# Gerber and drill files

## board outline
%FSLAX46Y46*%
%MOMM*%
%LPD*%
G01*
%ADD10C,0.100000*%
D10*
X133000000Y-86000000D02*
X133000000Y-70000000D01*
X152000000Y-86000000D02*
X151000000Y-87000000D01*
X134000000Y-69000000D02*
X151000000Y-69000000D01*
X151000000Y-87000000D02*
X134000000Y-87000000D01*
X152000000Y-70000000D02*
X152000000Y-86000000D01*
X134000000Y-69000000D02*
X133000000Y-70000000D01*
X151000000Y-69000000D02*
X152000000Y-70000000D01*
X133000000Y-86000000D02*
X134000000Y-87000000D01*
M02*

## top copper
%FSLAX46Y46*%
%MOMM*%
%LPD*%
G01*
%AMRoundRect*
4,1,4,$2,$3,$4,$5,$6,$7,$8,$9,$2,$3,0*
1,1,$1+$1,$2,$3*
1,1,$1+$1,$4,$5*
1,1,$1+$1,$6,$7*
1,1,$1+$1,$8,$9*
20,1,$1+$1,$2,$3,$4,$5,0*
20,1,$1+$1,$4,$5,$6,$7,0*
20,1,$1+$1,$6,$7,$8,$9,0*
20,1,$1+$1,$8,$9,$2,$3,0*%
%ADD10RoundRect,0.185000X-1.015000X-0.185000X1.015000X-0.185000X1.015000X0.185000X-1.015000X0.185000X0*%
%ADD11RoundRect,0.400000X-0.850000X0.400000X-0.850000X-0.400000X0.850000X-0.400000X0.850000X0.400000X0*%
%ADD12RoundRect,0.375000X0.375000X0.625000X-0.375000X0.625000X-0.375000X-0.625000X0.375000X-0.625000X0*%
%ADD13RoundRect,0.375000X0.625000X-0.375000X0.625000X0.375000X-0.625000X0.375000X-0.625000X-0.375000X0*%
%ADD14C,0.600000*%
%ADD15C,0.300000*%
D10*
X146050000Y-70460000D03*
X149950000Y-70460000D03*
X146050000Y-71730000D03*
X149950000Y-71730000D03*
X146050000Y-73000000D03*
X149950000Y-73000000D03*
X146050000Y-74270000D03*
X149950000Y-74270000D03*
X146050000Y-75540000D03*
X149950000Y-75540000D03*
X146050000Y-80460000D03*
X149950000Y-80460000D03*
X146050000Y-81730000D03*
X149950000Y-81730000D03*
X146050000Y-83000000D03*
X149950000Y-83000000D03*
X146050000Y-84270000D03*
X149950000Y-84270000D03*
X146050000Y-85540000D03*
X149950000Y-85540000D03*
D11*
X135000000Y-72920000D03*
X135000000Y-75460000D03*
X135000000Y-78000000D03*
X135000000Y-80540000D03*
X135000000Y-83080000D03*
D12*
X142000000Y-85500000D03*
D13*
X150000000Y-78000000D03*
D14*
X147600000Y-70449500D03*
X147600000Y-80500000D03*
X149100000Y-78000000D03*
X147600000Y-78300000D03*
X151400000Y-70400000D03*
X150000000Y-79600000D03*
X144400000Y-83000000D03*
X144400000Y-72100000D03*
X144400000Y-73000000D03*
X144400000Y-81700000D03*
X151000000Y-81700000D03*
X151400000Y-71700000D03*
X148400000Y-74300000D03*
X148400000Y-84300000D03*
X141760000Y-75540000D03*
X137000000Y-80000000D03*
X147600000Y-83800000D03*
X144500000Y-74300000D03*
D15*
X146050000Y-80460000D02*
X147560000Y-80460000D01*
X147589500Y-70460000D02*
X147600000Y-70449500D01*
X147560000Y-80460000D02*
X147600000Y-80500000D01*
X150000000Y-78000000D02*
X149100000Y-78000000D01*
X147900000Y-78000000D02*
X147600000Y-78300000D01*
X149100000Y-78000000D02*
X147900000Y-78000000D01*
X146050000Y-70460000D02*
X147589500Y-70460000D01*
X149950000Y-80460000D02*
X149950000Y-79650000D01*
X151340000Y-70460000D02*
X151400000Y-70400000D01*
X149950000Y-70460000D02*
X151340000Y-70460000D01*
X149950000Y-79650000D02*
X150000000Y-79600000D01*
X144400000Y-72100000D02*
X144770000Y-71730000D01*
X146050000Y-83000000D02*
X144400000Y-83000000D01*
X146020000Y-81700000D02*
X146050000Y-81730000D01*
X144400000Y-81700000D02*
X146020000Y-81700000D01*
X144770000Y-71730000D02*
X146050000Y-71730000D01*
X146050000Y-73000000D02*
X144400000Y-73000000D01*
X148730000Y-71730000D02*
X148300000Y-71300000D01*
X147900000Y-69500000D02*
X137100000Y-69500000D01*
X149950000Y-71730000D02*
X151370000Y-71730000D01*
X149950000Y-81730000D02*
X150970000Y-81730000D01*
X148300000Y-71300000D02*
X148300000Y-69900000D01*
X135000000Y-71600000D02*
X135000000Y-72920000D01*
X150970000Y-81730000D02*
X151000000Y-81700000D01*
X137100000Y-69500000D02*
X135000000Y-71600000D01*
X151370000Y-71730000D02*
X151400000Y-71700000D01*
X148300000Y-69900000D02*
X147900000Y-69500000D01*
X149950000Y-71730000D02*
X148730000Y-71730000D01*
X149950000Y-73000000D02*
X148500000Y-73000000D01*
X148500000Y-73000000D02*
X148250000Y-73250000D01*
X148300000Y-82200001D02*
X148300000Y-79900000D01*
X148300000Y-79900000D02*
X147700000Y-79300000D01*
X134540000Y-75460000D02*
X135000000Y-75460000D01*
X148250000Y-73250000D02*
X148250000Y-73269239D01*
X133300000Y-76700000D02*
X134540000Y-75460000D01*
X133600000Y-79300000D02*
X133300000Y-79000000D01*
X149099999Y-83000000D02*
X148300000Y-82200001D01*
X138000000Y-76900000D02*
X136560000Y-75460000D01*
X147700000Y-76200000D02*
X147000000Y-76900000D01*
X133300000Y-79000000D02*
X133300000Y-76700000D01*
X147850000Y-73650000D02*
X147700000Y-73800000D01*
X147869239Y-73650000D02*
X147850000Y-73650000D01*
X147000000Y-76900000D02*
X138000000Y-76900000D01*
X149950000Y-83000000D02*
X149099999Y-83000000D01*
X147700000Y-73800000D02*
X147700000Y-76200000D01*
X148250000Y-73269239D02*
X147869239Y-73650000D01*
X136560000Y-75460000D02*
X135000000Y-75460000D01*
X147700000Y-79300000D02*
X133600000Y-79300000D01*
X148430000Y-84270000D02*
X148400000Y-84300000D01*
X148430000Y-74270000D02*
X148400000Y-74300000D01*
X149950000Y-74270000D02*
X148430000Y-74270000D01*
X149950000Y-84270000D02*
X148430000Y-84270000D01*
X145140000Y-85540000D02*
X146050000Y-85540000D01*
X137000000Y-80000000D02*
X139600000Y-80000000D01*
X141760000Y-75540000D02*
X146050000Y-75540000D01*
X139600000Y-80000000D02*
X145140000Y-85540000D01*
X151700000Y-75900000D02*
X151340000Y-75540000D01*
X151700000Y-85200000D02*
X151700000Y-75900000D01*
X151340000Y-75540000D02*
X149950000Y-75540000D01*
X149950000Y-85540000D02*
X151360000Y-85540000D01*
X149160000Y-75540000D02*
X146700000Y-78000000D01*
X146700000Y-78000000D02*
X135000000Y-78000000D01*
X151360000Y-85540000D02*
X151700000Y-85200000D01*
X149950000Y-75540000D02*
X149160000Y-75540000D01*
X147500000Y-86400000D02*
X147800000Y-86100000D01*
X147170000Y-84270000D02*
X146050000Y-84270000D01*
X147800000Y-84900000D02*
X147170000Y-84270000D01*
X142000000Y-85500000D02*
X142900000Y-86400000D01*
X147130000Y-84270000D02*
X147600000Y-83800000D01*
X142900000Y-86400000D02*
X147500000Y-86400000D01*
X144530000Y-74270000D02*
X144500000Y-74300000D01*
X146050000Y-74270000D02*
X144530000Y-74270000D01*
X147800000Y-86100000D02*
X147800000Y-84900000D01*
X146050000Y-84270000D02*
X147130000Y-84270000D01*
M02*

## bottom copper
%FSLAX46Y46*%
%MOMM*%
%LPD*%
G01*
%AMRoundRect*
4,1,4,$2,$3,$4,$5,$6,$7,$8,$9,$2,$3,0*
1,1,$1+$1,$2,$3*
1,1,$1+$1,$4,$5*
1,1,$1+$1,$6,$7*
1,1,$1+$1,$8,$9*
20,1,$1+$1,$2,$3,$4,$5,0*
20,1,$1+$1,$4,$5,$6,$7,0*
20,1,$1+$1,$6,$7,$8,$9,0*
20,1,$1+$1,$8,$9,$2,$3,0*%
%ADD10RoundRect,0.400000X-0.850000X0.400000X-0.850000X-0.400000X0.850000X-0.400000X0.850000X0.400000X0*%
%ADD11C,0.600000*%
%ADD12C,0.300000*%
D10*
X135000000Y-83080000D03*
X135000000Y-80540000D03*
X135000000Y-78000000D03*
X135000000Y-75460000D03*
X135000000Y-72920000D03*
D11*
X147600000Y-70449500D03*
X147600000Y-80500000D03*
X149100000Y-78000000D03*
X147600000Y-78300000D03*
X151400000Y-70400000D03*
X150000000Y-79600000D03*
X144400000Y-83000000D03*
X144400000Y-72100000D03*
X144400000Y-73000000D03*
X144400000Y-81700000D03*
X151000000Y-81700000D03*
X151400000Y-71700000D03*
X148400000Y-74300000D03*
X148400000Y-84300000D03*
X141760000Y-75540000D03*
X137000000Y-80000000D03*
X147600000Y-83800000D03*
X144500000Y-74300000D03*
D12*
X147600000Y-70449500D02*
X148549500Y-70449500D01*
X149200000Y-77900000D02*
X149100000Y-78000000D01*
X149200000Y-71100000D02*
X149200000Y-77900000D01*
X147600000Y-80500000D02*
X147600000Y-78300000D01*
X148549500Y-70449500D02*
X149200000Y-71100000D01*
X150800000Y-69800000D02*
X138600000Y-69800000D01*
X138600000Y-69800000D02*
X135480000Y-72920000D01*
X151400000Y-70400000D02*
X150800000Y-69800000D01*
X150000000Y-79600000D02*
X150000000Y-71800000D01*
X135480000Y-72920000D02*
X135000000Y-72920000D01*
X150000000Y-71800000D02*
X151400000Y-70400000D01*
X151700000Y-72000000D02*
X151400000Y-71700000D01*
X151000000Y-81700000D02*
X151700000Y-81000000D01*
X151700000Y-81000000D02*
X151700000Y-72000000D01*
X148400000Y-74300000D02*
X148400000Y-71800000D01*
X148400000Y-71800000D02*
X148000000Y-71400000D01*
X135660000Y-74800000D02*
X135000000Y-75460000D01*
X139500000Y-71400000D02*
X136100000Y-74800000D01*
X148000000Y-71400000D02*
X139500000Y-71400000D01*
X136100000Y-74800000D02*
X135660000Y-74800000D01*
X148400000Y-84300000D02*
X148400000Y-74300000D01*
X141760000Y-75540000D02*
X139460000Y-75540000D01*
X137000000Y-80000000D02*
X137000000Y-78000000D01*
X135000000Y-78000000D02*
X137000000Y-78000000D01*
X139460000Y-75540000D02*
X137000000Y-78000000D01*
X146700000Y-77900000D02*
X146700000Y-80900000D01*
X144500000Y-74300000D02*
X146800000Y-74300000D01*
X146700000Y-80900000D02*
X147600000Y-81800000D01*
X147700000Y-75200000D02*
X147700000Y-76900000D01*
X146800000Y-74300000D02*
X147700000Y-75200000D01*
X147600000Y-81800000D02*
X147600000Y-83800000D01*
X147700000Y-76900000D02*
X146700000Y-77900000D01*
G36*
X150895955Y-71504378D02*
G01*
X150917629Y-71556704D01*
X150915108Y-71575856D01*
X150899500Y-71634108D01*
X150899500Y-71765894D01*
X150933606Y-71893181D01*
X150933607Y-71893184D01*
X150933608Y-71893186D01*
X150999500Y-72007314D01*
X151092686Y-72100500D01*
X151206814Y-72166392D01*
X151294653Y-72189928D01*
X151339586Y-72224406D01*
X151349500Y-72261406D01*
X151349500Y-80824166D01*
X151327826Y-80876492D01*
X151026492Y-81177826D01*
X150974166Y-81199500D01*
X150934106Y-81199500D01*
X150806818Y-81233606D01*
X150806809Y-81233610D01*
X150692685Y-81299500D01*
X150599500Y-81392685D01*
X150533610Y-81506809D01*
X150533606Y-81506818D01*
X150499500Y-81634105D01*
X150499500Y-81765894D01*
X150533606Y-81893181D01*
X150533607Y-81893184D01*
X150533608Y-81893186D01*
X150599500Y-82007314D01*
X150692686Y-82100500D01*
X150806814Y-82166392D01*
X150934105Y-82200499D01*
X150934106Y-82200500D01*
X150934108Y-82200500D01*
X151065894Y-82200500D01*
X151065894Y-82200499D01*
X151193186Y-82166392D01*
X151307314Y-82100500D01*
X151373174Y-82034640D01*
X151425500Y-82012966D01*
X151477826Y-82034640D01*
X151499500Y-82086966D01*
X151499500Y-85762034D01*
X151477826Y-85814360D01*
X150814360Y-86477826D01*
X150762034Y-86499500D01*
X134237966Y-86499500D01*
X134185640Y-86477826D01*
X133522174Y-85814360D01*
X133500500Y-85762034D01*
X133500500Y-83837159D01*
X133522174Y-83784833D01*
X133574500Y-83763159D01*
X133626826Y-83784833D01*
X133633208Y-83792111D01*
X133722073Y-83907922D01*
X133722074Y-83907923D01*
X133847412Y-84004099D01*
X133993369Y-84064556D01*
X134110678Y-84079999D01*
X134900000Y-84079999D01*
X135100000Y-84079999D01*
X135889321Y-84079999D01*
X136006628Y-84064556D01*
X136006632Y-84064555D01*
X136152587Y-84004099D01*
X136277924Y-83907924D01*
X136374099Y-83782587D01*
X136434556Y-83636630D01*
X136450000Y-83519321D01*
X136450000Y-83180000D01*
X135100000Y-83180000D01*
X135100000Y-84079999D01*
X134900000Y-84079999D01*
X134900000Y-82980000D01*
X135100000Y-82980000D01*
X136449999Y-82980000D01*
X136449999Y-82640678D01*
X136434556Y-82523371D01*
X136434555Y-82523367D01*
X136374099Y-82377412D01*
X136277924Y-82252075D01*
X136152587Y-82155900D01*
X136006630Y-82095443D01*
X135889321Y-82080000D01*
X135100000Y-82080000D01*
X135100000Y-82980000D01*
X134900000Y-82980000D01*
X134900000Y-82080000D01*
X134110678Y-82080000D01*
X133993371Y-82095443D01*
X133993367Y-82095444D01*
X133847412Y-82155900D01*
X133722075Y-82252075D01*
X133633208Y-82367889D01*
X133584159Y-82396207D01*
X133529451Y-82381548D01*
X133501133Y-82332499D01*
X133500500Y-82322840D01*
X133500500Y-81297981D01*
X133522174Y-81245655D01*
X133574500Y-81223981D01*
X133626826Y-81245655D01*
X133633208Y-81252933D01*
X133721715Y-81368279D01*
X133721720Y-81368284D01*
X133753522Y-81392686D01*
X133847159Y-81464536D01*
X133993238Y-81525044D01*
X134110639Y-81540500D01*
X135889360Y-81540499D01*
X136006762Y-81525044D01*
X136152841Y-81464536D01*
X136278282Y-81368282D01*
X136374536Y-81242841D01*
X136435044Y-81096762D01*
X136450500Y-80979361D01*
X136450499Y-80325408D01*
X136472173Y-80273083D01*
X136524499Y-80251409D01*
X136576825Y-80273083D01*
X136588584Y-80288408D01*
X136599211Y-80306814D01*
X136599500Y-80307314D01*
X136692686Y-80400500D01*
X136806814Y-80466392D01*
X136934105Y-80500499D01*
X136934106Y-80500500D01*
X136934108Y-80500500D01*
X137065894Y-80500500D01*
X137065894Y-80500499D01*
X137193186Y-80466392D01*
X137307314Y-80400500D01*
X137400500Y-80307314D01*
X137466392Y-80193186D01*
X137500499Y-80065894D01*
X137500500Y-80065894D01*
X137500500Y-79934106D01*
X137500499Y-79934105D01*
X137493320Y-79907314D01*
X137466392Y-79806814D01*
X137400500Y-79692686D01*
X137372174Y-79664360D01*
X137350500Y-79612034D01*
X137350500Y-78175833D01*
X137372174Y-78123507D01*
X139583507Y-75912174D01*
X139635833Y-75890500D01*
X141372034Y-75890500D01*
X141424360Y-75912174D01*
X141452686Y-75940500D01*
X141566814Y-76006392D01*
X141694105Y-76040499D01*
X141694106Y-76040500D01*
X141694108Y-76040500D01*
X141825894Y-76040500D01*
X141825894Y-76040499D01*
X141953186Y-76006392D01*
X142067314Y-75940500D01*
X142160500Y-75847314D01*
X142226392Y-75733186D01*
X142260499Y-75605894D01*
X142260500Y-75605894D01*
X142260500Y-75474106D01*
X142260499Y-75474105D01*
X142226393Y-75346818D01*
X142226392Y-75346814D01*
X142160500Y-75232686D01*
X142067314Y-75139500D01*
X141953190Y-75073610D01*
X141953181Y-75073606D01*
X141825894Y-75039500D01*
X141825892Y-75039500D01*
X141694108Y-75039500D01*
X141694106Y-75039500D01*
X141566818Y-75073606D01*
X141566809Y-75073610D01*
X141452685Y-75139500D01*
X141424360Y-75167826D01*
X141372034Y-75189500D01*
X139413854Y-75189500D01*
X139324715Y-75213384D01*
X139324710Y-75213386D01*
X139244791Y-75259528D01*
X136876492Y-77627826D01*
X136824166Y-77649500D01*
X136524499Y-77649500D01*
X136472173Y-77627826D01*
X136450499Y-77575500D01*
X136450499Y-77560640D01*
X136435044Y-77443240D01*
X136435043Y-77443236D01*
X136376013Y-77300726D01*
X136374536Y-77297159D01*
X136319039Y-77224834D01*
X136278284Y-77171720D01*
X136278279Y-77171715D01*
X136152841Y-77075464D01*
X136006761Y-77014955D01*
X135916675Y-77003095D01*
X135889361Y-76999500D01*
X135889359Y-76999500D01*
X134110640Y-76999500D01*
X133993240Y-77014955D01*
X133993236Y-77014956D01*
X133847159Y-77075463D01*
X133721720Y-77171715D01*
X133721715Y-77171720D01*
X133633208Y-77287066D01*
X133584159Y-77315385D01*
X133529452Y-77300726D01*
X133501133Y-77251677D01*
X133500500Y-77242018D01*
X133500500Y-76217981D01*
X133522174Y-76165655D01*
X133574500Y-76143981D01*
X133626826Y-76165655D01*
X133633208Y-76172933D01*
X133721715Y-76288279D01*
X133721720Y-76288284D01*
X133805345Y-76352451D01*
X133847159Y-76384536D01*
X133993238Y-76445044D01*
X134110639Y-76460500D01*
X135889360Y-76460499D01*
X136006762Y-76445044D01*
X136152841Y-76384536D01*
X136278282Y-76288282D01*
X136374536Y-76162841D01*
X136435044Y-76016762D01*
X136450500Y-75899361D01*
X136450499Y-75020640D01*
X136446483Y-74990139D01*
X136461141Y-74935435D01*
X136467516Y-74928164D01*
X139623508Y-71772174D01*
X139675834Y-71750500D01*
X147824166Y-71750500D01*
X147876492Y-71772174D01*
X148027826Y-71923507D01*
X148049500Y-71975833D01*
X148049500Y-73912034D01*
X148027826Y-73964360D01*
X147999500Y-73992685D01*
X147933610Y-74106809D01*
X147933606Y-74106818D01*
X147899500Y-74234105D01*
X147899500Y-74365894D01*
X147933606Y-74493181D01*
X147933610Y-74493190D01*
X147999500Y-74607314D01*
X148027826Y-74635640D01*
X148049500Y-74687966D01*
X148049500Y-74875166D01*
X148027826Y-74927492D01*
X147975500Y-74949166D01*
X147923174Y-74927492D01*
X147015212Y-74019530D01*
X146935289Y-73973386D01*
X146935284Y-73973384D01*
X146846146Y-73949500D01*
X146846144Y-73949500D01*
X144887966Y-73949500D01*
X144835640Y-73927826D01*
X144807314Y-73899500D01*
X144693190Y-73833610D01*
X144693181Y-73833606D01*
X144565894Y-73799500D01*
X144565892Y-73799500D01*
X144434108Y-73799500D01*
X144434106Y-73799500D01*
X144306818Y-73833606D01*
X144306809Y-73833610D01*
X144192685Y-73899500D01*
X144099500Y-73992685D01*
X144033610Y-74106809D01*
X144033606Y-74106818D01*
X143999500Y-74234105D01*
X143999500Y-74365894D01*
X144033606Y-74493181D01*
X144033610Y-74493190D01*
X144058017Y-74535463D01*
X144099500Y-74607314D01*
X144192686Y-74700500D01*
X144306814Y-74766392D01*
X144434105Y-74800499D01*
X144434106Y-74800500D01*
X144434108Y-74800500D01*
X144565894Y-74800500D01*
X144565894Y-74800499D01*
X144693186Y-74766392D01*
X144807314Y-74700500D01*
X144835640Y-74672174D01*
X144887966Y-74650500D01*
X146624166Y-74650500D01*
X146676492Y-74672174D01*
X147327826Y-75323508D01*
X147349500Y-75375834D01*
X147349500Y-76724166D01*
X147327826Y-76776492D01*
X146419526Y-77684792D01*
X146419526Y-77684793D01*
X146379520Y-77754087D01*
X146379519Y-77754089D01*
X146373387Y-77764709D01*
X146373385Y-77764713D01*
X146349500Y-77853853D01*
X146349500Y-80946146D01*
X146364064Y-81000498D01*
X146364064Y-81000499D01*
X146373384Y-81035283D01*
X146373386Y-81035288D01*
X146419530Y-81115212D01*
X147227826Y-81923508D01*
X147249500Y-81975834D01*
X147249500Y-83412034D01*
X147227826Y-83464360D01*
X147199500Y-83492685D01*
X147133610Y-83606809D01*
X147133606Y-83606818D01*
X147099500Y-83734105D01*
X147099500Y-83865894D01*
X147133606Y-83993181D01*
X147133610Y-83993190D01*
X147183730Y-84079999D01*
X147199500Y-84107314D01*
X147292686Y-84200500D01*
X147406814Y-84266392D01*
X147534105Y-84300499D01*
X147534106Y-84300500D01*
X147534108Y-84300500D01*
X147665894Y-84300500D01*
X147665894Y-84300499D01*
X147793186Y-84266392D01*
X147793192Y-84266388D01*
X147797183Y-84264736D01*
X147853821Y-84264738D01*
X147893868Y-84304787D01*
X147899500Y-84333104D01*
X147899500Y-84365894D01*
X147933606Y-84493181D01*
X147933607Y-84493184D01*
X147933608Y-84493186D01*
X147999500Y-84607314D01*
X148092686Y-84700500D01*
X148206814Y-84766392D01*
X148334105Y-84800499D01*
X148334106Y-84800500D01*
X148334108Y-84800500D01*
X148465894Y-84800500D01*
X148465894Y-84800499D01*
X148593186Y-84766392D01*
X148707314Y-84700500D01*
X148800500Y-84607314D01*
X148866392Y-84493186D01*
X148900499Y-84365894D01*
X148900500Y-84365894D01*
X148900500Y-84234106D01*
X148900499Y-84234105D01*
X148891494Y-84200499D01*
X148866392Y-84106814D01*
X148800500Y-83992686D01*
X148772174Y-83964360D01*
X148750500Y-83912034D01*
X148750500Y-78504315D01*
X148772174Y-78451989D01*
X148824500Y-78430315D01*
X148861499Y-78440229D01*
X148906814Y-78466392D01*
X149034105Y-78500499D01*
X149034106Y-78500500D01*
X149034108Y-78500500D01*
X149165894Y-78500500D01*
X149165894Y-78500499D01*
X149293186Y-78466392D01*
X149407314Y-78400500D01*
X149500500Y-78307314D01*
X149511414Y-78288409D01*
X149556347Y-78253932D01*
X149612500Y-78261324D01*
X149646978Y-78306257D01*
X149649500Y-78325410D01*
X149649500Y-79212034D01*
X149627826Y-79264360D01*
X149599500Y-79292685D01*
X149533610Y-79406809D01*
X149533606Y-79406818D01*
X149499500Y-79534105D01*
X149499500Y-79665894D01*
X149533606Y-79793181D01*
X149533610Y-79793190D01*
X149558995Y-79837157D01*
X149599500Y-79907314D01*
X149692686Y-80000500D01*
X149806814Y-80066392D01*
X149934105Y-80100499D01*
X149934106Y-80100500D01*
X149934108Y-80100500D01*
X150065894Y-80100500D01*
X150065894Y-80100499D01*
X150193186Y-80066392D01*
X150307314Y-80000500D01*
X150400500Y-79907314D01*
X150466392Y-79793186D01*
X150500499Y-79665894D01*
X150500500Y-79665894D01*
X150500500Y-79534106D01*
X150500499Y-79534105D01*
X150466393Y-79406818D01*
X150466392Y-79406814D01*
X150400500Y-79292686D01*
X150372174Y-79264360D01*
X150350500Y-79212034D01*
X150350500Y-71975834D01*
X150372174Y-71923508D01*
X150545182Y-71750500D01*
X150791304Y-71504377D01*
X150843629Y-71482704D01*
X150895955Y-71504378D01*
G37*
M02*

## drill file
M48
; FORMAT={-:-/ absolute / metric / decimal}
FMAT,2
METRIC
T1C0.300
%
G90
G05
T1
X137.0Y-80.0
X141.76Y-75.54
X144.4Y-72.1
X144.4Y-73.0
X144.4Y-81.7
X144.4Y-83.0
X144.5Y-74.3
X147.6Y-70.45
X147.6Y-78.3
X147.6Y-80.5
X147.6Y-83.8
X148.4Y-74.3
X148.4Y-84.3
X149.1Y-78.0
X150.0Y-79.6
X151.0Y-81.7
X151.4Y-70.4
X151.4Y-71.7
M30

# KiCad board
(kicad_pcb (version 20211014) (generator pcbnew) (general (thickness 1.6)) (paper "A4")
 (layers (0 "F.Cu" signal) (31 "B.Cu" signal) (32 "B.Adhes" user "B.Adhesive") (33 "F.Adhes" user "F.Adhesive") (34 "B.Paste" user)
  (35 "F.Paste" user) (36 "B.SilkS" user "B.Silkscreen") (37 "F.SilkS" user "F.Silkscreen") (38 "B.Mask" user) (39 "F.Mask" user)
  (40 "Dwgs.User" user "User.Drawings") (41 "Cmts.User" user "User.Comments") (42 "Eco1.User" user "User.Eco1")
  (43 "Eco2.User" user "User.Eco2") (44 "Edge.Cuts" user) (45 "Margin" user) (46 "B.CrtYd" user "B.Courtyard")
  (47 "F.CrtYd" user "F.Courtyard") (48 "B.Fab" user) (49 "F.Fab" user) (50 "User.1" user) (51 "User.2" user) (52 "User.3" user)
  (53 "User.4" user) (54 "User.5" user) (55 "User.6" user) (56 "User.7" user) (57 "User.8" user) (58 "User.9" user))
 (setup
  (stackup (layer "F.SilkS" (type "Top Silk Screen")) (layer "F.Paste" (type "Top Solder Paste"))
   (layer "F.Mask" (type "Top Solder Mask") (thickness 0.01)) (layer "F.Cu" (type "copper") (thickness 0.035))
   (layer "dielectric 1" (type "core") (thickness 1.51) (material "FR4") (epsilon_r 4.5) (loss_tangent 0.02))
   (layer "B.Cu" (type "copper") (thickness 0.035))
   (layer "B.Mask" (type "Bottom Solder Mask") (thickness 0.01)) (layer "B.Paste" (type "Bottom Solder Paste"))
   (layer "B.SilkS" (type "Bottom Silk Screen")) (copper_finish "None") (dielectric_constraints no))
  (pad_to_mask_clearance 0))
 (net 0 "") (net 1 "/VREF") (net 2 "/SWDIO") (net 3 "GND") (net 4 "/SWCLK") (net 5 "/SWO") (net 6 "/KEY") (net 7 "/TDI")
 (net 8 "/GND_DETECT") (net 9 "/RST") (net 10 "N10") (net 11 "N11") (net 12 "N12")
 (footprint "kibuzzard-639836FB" (layer "F.Cu") (at 142 81.8 90)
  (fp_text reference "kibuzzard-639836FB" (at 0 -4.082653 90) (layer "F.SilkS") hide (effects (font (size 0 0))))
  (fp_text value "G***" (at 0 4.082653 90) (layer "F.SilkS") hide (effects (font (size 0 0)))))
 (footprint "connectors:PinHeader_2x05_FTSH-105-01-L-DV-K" (layer "F.Cu") (at 148 73)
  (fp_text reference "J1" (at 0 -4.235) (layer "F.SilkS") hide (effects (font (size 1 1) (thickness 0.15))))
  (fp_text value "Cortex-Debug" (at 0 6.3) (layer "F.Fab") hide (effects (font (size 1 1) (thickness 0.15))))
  (pad "1" smd roundrect (at -1.95 -2.54) (size 2.4 0.74) (layers "F.Cu" "F.Paste" "F.Mask") (roundrect_rratio 0.25) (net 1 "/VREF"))
  (pad "2" smd roundrect (at 1.95 -2.54) (size 2.4 0.74) (layers "F.Cu" "F.Paste" "F.Mask") (roundrect_rratio 0.25) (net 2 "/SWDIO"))
  (pad "3" smd roundrect (at -1.95 -1.27) (size 2.4 0.74) (layers "F.Cu" "F.Paste" "F.Mask") (roundrect_rratio 0.25) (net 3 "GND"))
  (pad "4" smd roundrect (at 1.95 -1.27) (size 2.4 0.74) (layers "F.Cu" "F.Paste" "F.Mask") (roundrect_rratio 0.25) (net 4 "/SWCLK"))
  (pad "5" smd roundrect (at -1.95 0) (size 2.4 0.74) (layers "F.Cu" "F.Paste" "F.Mask") (roundrect_rratio 0.25) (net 3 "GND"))
  (pad "6" smd roundrect (at 1.95 0) (size 2.4 0.74) (layers "F.Cu" "F.Paste" "F.Mask") (roundrect_rratio 0.25) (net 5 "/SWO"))
  (pad "7" smd roundrect (at -1.95 1.27) (size 2.4 0.74) (layers "F.Cu" "F.Paste" "F.Mask") (roundrect_rratio 0.25) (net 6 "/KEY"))
  (pad "8" smd roundrect (at 1.95 1.27) (size 2.4 0.74) (layers "F.Cu" "F.Paste" "F.Mask") (roundrect_rratio 0.25) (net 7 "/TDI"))
  (pad "9" smd roundrect (at -1.95 2.54) (size 2.4 0.74) (layers "F.Cu" "F.Paste" "F.Mask") (roundrect_rratio 0.25) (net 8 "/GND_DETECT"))
  (pad "10" smd roundrect (at 1.95 2.54) (size 2.4 0.74) (layers "F.Cu" "F.Paste" "F.Mask") (roundrect_rratio 0.25) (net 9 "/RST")))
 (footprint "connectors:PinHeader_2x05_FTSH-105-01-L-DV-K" (layer "F.Cu") (at 148 83)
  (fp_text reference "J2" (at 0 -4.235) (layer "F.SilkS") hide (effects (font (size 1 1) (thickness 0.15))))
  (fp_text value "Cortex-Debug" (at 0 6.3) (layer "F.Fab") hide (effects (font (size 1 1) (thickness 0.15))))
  (pad "1" smd roundrect (at -1.95 -2.54) (size 2.4 0.74) (layers "F.Cu" "F.Paste" "F.Mask") (roundrect_rratio 0.25) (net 1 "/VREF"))
  (pad "2" smd roundrect (at 1.95 -2.54) (size 2.4 0.74) (layers "F.Cu" "F.Paste" "F.Mask") (roundrect_rratio 0.25) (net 2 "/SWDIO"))
  (pad "3" smd roundrect (at -1.95 -1.27) (size 2.4 0.74) (layers "F.Cu" "F.Paste" "F.Mask") (roundrect_rratio 0.25) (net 3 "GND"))
  (pad "4" smd roundrect (at 1.95 -1.27) (size 2.4 0.74) (layers "F.Cu" "F.Paste" "F.Mask") (roundrect_rratio 0.25) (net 4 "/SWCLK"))
  (pad "5" smd roundrect (at -1.95 0) (size 2.4 0.74) (layers "F.Cu" "F.Paste" "F.Mask") (roundrect_rratio 0.25) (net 3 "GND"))
  (pad "6" smd roundrect (at 1.95 0) (size 2.4 0.74) (layers "F.Cu" "F.Paste" "F.Mask") (roundrect_rratio 0.25) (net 5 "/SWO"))
  (pad "7" smd roundrect (at -1.95 1.27) (size 2.4 0.74) (layers "F.Cu" "F.Paste" "F.Mask") (roundrect_rratio 0.25) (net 6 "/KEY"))
  (pad "8" smd roundrect (at 1.95 1.27) (size 2.4 0.74) (layers "F.Cu" "F.Paste" "F.Mask") (roundrect_rratio 0.25) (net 7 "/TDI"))
  (pad "9" smd roundrect (at -1.95 2.54) (size 2.4 0.74) (layers "F.Cu" "F.Paste" "F.Mask") (roundrect_rratio 0.25) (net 8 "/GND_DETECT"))
  (pad "10" smd roundrect (at 1.95 2.54) (size 2.4 0.74) (layers "F.Cu" "F.Paste" "F.Mask") (roundrect_rratio 0.25) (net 9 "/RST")))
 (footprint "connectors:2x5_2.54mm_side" (layer "F.Cu") (at 135 78 -90)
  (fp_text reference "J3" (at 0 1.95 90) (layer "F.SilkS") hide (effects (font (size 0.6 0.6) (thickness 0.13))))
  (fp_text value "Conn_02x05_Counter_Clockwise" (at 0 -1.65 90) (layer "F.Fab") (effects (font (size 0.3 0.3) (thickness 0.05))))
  (pad "1" smd roundrect locked (at -5.08 0 270) (size 1.6 2.5) (layers "F.Cu" "F.Mask") (roundrect_rratio 0.25) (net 4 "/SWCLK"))
  (pad "2" smd roundrect locked (at -2.54 0 270) (size 1.6 2.5) (layers "F.Cu" "F.Mask") (roundrect_rratio 0.25) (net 5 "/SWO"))
  (pad "3" smd roundrect locked (at 0 0 270) (size 1.6 2.5) (layers "F.Cu" "F.Mask") (roundrect_rratio 0.25) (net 9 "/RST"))
  (pad "4" smd roundrect locked (at 2.54 0 270) (size 1.6 2.5) (layers "F.Cu" "F.Mask") (roundrect_rratio 0.25) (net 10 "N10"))
  (pad "5" smd roundrect locked (at 5.08 0 270) (size 1.6 2.5) (layers "F.Cu" "F.Mask") (roundrect_rratio 0.25) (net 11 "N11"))
  (pad "6" smd roundrect locked (at 5.08 0 270) (size 1.6 2.5) (layers "B.Cu" "B.Mask") (roundrect_rratio 0.25) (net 3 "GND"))
  (pad "7" smd roundrect locked (at 2.54 0 270) (size 1.6 2.5) (layers "B.Cu" "B.Mask") (roundrect_rratio 0.25) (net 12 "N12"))
  (pad "8" smd roundrect locked (at 0 0 270) (size 1.6 2.5) (layers "B.Cu" "B.Mask") (roundrect_rratio 0.25) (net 8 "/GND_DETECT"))
  (pad "9" smd roundrect locked (at -2.54 0 270) (size 1.6 2.5) (layers "B.Cu" "B.Mask") (roundrect_rratio 0.25) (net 7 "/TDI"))
  (pad "10" smd roundrect locked (at -5.08 0 270) (size 1.6 2.5) (layers "B.Cu" "B.Mask") (roundrect_rratio 0.25) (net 2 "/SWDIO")))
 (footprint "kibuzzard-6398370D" (layer "F.Cu") (at 145.7 78)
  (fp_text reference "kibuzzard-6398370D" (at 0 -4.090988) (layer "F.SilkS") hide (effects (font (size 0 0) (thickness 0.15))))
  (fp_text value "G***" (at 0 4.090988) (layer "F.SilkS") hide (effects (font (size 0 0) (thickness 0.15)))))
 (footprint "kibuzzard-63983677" (layer "F.Cu") (at 140.1 72.9)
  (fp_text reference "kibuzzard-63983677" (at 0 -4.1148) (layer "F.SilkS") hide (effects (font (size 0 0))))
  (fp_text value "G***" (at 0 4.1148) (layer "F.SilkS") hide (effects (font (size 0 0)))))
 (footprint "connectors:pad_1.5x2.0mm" (layer "F.Cu") (at 142 85.5 180)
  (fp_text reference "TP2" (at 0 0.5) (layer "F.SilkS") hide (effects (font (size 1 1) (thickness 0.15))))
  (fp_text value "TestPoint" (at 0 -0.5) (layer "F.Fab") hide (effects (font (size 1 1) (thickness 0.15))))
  (pad "1" smd roundrect locked (at 0 0 180) (size 1.5 2) (layers "F.Cu" "F.Mask") (roundrect_rratio 0.25) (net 6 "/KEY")))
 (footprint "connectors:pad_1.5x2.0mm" (layer "F.Cu") (at 150 78 90)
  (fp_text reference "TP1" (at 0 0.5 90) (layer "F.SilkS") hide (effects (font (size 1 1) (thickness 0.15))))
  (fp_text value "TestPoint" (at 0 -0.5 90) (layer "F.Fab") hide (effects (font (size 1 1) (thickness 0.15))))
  (pad "1" smd roundrect locked (at 0 0 90) (size 1.5 2) (layers "F.Cu" "F.Mask") (roundrect_rratio 0.25) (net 1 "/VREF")))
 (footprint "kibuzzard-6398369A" (layer "F.Cu") (at 138.9 78)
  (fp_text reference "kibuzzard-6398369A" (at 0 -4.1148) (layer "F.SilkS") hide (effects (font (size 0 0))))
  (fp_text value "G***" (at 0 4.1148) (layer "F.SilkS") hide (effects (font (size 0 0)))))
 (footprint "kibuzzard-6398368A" (layer "F.Cu") (at 138.9 75.5)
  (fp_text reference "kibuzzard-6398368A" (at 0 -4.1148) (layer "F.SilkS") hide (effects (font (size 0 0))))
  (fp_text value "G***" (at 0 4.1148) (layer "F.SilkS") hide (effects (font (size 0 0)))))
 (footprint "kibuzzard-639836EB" (layer "B.Cu") (at 138.9 83.1)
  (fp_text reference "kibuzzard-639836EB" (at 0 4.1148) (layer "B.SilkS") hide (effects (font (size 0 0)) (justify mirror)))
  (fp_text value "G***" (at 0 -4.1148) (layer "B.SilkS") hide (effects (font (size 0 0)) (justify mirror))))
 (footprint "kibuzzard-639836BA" (layer "B.Cu") (at 138.9 75.5)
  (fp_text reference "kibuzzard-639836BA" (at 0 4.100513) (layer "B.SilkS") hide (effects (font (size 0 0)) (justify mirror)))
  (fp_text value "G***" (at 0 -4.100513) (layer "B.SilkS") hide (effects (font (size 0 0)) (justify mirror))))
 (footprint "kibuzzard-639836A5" (layer "B.Cu") (at 140.1 72.9)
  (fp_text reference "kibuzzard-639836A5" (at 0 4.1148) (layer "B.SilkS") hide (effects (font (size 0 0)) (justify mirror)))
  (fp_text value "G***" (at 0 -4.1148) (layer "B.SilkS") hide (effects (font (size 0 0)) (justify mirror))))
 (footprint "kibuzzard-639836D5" (layer "B.Cu") (at 141.3 78)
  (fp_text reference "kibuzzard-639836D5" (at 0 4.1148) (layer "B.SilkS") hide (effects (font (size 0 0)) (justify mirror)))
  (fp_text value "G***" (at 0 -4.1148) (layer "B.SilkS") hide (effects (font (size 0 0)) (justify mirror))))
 (gr_line (start 133 86) (end 133 70) (layer "Edge.Cuts") (width 0.1))
 (gr_line (start 152 86) (end 151 87) (layer "Edge.Cuts") (width 0.1))
 (gr_line (start 134 69) (end 151 69) (layer "Edge.Cuts") (width 0.1))
 (gr_line (start 151 87) (end 134 87) (layer "Edge.Cuts") (width 0.1))
 (gr_line (start 152 70) (end 152 86) (layer "Edge.Cuts") (width 0.1))
 (gr_line (start 134 69) (end 133 70) (layer "Edge.Cuts") (width 0.1))
 (gr_line (start 151 69) (end 152 70) (layer "Edge.Cuts") (width 0.1))
 (gr_line (start 133 86) (end 134 87) (layer "Edge.Cuts") (width 0.1))
 (segment (start 146.05 80.46) (end 147.56 80.46) (width 0.3) (layer "F.Cu") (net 1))
 (segment (start 147.5895 70.46) (end 147.6 70.4495) (width 0.3) (layer "F.Cu") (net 1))
 (segment (start 147.56 80.46) (end 147.6 80.5) (width 0.3) (layer "F.Cu") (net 1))
 (segment (start 150 78) (end 149.1 78) (width 0.3) (layer "F.Cu") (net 1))
 (segment (start 147.9 78) (end 147.6 78.3) (width 0.3) (layer "F.Cu") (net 1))
 (segment (start 149.1 78) (end 147.9 78) (width 0.3) (layer "F.Cu") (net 1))
 (segment (start 146.05 70.46) (end 147.5895 70.46) (width 0.3) (layer "F.Cu") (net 1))
 (via (at 147.6 70.4495) (size 0.6) (drill 0.3) (layers "F.Cu" "B.Cu") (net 1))
 (via (at 147.6 80.5) (size 0.6) (drill 0.3) (layers "F.Cu" "B.Cu") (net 1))
 (via (at 149.1 78) (size 0.6) (drill 0.3) (layers "F.Cu" "B.Cu") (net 1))
 (via (at 147.6 78.3) (size 0.6) (drill 0.3) (layers "F.Cu" "B.Cu") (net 1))
 (segment (start 147.6 70.4495) (end 148.5495 70.4495) (width 0.3) (layer "B.Cu") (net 1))
 (segment (start 149.2 77.9) (end 149.1 78) (width 0.3) (layer "B.Cu") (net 1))
 (segment (start 149.2 71.1) (end 149.2 77.9) (width 0.3) (layer "B.Cu") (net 1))
 (segment (start 147.6 80.5) (end 147.6 78.3) (width 0.3) (layer "B.Cu") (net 1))
 (segment (start 148.5495 70.4495) (end 149.2 71.1) (width 0.3) (layer "B.Cu") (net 1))
 (segment (start 149.95 80.46) (end 149.95 79.65) (width 0.3) (layer "F.Cu") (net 2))
 (segment (start 151.34 70.46) (end 151.4 70.4) (width 0.3) (layer "F.Cu") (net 2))
 (segment (start 149.95 70.46) (end 151.34 70.46) (width 0.3) (layer "F.Cu") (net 2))
 (segment (start 149.95 79.65) (end 150 79.6) (width 0.3) (layer "F.Cu") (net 2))
 (via (at 151.4 70.4) (size 0.6) (drill 0.3) (layers "F.Cu" "B.Cu") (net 2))
 (via (at 150 79.6) (size 0.6) (drill 0.3) (layers "F.Cu" "B.Cu") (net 2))
 (segment (start 150.8 69.8) (end 138.6 69.8) (width 0.3) (layer "B.Cu") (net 2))
 (segment (start 138.6 69.8) (end 135.48 72.92) (width 0.3) (layer "B.Cu") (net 2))
 (segment (start 151.4 70.4) (end 150.8 69.8) (width 0.3) (layer "B.Cu") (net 2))
 (segment (start 150 79.6) (end 150 71.8) (width 0.3) (layer "B.Cu") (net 2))
 (segment (start 135.48 72.92) (end 135 72.92) (width 0.3) (layer "B.Cu") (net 2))
 (segment (start 150 71.8) (end 151.4 70.4) (width 0.3) (layer "B.Cu") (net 2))
 (segment (start 144.4 72.1) (end 144.77 71.73) (width 0.3) (layer "F.Cu") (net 3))
 (segment (start 146.05 83) (end 144.4 83) (width 0.3) (layer "F.Cu") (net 3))
 (segment (start 146.02 81.7) (end 146.05 81.73) (width 0.3) (layer "F.Cu") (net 3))
 (segment (start 144.4 81.7) (end 146.02 81.7) (width 0.3) (layer "F.Cu") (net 3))
 (segment (start 144.77 71.73) (end 146.05 71.73) (width 0.3) (layer "F.Cu") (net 3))
 (segment (start 146.05 73) (end 144.4 73) (width 0.3) (layer "F.Cu") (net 3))
 (via (at 144.4 83) (size 0.6) (drill 0.3) (layers "F.Cu" "B.Cu") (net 3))
 (via (at 144.4 72.1) (size 0.6) (drill 0.3) (layers "F.Cu" "B.Cu") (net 3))
 (via (at 144.4 73) (size 0.6) (drill 0.3) (layers "F.Cu" "B.Cu") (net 3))
 (via (at 144.4 81.7) (size 0.6) (drill 0.3) (layers "F.Cu" "B.Cu") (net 3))
 (segment (start 148.73 71.73) (end 148.3 71.3) (width 0.3) (layer "F.Cu") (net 4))
 (segment (start 147.9 69.5) (end 137.1 69.5) (width 0.3) (layer "F.Cu") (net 4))
 (segment (start 149.95 71.73) (end 151.37 71.73) (width 0.3) (layer "F.Cu") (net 4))
 (segment (start 149.95 81.73) (end 150.97 81.73) (width 0.3) (layer "F.Cu") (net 4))
 (segment (start 148.3 71.3) (end 148.3 69.9) (width 0.3) (layer "F.Cu") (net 4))
 (segment (start 135 71.6) (end 135 72.92) (width 0.3) (layer "F.Cu") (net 4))
 (segment (start 150.97 81.73) (end 151 81.7) (width 0.3) (layer "F.Cu") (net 4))
 (segment (start 137.1 69.5) (end 135 71.6) (width 0.3) (layer "F.Cu") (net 4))
 (segment (start 151.37 71.73) (end 151.4 71.7) (width 0.3) (layer "F.Cu") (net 4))
 (segment (start 148.3 69.9) (end 147.9 69.5) (width 0.3) (layer "F.Cu") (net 4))
 (segment (start 149.95 71.73) (end 148.73 71.73) (width 0.3) (layer "F.Cu") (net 4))
 (via (at 151 81.7) (size 0.6) (drill 0.3) (layers "F.Cu" "B.Cu") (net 4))
 (via (at 151.4 71.7) (size 0.6) (drill 0.3) (layers "F.Cu" "B.Cu") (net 4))
 (segment (start 151.7 72) (end 151.4 71.7) (width 0.3) (layer "B.Cu") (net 4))
 (segment (start 151 81.7) (end 151.7 81) (width 0.3) (layer "B.Cu") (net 4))
 (segment (start 151.7 81) (end 151.7 72) (width 0.3) (layer "B.Cu") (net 4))
 (segment (start 149.95 73) (end 148.5 73) (width 0.3) (layer "F.Cu") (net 5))
 (segment (start 148.5 73) (end 148.25 73.25) (width 0.3) (layer "F.Cu") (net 5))
 (segment (start 148.3 82.200001) (end 148.3 79.9) (width 0.3) (layer "F.Cu") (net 5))
 (segment (start 148.3 79.9) (end 147.7 79.3) (width 0.3) (layer "F.Cu") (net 5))
 (segment (start 134.54 75.46) (end 135 75.46) (width 0.3) (layer "F.Cu") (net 5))
 (segment (start 148.25 73.25) (end 148.25 73.269239) (width 0.3) (layer "F.Cu") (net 5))
 (segment (start 133.3 76.7) (end 134.54 75.46) (width 0.3) (layer "F.Cu") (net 5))
 (segment (start 133.6 79.3) (end 133.3 79) (width 0.3) (layer "F.Cu") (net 5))
 (segment (start 149.099999 83) (end 148.3 82.200001) (width 0.3) (layer "F.Cu") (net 5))
 (segment (start 138 76.9) (end 136.56 75.46) (width 0.3) (layer "F.Cu") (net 5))
 (segment (start 147.7 76.2) (end 147 76.9) (width 0.3) (layer "F.Cu") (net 5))
 (segment (start 133.3 79) (end 133.3 76.7) (width 0.3) (layer "F.Cu") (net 5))
 (segment (start 147.85 73.65) (end 147.7 73.8) (width 0.3) (layer "F.Cu") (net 5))
 (segment (start 147.869239 73.65) (end 147.85 73.65) (width 0.3) (layer "F.Cu") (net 5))
 (segment (start 147 76.9) (end 138 76.9) (width 0.3) (layer "F.Cu") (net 5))
 (segment (start 149.95 83) (end 149.099999 83) (width 0.3) (layer "F.Cu") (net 5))
 (segment (start 147.7 73.8) (end 147.7 76.2) (width 0.3) (layer "F.Cu") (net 5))
 (segment (start 148.25 73.269239) (end 147.869239 73.65) (width 0.3) (layer "F.Cu") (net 5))
 (segment (start 136.56 75.46) (end 135 75.46) (width 0.3) (layer "F.Cu") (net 5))
 (segment (start 147.7 79.3) (end 133.6 79.3) (width 0.3) (layer "F.Cu") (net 5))
 (segment (start 148.43 84.27) (end 148.4 84.3) (width 0.3) (layer "F.Cu") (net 7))
 (segment (start 148.43 74.27) (end 148.4 74.3) (width 0.3) (layer "F.Cu") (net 7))
 (segment (start 149.95 74.27) (end 148.43 74.27) (width 0.3) (layer "F.Cu") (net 7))
 (segment (start 149.95 84.27) (end 148.43 84.27) (width 0.3) (layer "F.Cu") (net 7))
 (via (at 148.4 74.3) (size 0.6) (drill 0.3) (layers "F.Cu" "B.Cu") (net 7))
 (via (at 148.4 84.3) (size 0.6) (drill 0.3) (layers "F.Cu" "B.Cu") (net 7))
 (segment (start 148.4 74.3) (end 148.4 71.8) (width 0.3) (layer "B.Cu") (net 7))
 (segment (start 148.4 71.8) (end 148 71.4) (width 0.3) (layer "B.Cu") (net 7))
 (segment (start 135.66 74.8) (end 135 75.46) (width 0.3) (layer "B.Cu") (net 7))
 (segment (start 139.5 71.4) (end 136.1 74.8) (width 0.3) (layer "B.Cu") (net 7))
 (segment (start 148 71.4) (end 139.5 71.4) (width 0.3) (layer "B.Cu") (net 7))
 (segment (start 136.1 74.8) (end 135.66 74.8) (width 0.3) (layer "B.Cu") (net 7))
 (segment (start 148.4 84.3) (end 148.4 74.3) (width 0.3) (layer "B.Cu") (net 7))
 (segment (start 145.14 85.54) (end 146.05 85.54) (width 0.3) (layer "F.Cu") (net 8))
 (segment (start 137 80) (end 139.6 80) (width 0.3) (layer "F.Cu") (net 8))
 (segment (start 141.76 75.54) (end 146.05 75.54) (width 0.3) (layer "F.Cu") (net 8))
 (segment (start 139.6 80) (end 145.14 85.54) (width 0.3) (layer "F.Cu") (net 8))
 (via (at 141.76 75.54) (size 0.6) (drill 0.3) (layers "F.Cu" "B.Cu") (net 8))
 (via (at 137 80) (size 0.6) (drill 0.3) (layers "F.Cu" "B.Cu") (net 8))
 (segment (start 141.76 75.54) (end 139.46 75.54) (width 0.3) (layer "B.Cu") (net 8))
 (segment (start 137 80) (end 137 78) (width 0.3) (layer "B.Cu") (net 8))
 (segment (start 135 78) (end 137 78) (width 0.3) (layer "B.Cu") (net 8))
 (segment (start 139.46 75.54) (end 137 78) (width 0.3) (layer "B.Cu") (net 8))
 (segment (start 151.7 75.9) (end 151.34 75.54) (width 0.3) (layer "F.Cu") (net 9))
 (segment (start 151.7 85.2) (end 151.7 75.9) (width 0.3) (layer "F.Cu") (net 9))
 (segment (start 151.34 75.54) (end 149.95 75.54) (width 0.3) (layer "F.Cu") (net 9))
 (segment (start 149.95 85.54) (end 151.36 85.54) (width 0.3) (layer "F.Cu") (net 9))
 (segment (start 149.16 75.54) (end 146.7 78) (width 0.3) (layer "F.Cu") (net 9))
 (segment (start 146.7 78) (end 135 78) (width 0.3) (layer "F.Cu") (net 9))
 (segment (start 151.36 85.54) (end 151.7 85.2) (width 0.3) (layer "F.Cu") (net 9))
 (segment (start 149.95 75.54) (end 149.16 75.54) (width 0.3) (layer "F.Cu") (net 9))
 (segment (start 147.5 86.4) (end 147.8 86.1) (width 0.3) (layer "F.Cu") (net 6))
 (segment (start 147.17 84.27) (end 146.05 84.27) (width 0.3) (layer "F.Cu") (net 6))
 (segment (start 147.8 84.9) (end 147.17 84.27) (width 0.3) (layer "F.Cu") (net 6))
 (segment (start 142 85.5) (end 142.9 86.4) (width 0.3) (layer "F.Cu") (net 6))
 (segment (start 147.13 84.27) (end 147.6 83.8) (width 0.3) (layer "F.Cu") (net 6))
 (segment (start 142.9 86.4) (end 147.5 86.4) (width 0.3) (layer "F.Cu") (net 6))
 (segment (start 144.53 74.27) (end 144.5 74.3) (width 0.3) (layer "F.Cu") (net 6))
 (segment (start 146.05 74.27) (end 144.53 74.27) (width 0.3) (layer "F.Cu") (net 6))
 (segment (start 147.8 86.1) (end 147.8 84.9) (width 0.3) (layer "F.Cu") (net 6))
 (segment (start 146.05 84.27) (end 147.13 84.27) (width 0.3) (layer "F.Cu") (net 6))
 (via (at 147.6 83.8) (size 0.6) (drill 0.3) (layers "F.Cu" "B.Cu") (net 6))
 (via (at 144.5 74.3) (size 0.6) (drill 0.3) (layers "F.Cu" "B.Cu") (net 6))
 (segment (start 146.7 77.9) (end 146.7 80.9) (width 0.3) (layer "B.Cu") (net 6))
 (segment (start 144.5 74.3) (end 146.8 74.3) (width 0.3) (layer "B.Cu") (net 6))
 (segment (start 146.7 80.9) (end 147.6 81.8) (width 0.3) (layer "B.Cu") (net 6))
 (segment (start 147.7 75.2) (end 147.7 76.9) (width 0.3) (layer "B.Cu") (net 6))
 (segment (start 146.8 74.3) (end 147.7 75.2) (width 0.3) (layer "B.Cu") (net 6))
 (segment (start 147.6 81.8) (end 147.6 83.8) (width 0.3) (layer "B.Cu") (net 6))
 (segment (start 147.7 76.9) (end 146.7 77.9) (width 0.3) (layer "B.Cu") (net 6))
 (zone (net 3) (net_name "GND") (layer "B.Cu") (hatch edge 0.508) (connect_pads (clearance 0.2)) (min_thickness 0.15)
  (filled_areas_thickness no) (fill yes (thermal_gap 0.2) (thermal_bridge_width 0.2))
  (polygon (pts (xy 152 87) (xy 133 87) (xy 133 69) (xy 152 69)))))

